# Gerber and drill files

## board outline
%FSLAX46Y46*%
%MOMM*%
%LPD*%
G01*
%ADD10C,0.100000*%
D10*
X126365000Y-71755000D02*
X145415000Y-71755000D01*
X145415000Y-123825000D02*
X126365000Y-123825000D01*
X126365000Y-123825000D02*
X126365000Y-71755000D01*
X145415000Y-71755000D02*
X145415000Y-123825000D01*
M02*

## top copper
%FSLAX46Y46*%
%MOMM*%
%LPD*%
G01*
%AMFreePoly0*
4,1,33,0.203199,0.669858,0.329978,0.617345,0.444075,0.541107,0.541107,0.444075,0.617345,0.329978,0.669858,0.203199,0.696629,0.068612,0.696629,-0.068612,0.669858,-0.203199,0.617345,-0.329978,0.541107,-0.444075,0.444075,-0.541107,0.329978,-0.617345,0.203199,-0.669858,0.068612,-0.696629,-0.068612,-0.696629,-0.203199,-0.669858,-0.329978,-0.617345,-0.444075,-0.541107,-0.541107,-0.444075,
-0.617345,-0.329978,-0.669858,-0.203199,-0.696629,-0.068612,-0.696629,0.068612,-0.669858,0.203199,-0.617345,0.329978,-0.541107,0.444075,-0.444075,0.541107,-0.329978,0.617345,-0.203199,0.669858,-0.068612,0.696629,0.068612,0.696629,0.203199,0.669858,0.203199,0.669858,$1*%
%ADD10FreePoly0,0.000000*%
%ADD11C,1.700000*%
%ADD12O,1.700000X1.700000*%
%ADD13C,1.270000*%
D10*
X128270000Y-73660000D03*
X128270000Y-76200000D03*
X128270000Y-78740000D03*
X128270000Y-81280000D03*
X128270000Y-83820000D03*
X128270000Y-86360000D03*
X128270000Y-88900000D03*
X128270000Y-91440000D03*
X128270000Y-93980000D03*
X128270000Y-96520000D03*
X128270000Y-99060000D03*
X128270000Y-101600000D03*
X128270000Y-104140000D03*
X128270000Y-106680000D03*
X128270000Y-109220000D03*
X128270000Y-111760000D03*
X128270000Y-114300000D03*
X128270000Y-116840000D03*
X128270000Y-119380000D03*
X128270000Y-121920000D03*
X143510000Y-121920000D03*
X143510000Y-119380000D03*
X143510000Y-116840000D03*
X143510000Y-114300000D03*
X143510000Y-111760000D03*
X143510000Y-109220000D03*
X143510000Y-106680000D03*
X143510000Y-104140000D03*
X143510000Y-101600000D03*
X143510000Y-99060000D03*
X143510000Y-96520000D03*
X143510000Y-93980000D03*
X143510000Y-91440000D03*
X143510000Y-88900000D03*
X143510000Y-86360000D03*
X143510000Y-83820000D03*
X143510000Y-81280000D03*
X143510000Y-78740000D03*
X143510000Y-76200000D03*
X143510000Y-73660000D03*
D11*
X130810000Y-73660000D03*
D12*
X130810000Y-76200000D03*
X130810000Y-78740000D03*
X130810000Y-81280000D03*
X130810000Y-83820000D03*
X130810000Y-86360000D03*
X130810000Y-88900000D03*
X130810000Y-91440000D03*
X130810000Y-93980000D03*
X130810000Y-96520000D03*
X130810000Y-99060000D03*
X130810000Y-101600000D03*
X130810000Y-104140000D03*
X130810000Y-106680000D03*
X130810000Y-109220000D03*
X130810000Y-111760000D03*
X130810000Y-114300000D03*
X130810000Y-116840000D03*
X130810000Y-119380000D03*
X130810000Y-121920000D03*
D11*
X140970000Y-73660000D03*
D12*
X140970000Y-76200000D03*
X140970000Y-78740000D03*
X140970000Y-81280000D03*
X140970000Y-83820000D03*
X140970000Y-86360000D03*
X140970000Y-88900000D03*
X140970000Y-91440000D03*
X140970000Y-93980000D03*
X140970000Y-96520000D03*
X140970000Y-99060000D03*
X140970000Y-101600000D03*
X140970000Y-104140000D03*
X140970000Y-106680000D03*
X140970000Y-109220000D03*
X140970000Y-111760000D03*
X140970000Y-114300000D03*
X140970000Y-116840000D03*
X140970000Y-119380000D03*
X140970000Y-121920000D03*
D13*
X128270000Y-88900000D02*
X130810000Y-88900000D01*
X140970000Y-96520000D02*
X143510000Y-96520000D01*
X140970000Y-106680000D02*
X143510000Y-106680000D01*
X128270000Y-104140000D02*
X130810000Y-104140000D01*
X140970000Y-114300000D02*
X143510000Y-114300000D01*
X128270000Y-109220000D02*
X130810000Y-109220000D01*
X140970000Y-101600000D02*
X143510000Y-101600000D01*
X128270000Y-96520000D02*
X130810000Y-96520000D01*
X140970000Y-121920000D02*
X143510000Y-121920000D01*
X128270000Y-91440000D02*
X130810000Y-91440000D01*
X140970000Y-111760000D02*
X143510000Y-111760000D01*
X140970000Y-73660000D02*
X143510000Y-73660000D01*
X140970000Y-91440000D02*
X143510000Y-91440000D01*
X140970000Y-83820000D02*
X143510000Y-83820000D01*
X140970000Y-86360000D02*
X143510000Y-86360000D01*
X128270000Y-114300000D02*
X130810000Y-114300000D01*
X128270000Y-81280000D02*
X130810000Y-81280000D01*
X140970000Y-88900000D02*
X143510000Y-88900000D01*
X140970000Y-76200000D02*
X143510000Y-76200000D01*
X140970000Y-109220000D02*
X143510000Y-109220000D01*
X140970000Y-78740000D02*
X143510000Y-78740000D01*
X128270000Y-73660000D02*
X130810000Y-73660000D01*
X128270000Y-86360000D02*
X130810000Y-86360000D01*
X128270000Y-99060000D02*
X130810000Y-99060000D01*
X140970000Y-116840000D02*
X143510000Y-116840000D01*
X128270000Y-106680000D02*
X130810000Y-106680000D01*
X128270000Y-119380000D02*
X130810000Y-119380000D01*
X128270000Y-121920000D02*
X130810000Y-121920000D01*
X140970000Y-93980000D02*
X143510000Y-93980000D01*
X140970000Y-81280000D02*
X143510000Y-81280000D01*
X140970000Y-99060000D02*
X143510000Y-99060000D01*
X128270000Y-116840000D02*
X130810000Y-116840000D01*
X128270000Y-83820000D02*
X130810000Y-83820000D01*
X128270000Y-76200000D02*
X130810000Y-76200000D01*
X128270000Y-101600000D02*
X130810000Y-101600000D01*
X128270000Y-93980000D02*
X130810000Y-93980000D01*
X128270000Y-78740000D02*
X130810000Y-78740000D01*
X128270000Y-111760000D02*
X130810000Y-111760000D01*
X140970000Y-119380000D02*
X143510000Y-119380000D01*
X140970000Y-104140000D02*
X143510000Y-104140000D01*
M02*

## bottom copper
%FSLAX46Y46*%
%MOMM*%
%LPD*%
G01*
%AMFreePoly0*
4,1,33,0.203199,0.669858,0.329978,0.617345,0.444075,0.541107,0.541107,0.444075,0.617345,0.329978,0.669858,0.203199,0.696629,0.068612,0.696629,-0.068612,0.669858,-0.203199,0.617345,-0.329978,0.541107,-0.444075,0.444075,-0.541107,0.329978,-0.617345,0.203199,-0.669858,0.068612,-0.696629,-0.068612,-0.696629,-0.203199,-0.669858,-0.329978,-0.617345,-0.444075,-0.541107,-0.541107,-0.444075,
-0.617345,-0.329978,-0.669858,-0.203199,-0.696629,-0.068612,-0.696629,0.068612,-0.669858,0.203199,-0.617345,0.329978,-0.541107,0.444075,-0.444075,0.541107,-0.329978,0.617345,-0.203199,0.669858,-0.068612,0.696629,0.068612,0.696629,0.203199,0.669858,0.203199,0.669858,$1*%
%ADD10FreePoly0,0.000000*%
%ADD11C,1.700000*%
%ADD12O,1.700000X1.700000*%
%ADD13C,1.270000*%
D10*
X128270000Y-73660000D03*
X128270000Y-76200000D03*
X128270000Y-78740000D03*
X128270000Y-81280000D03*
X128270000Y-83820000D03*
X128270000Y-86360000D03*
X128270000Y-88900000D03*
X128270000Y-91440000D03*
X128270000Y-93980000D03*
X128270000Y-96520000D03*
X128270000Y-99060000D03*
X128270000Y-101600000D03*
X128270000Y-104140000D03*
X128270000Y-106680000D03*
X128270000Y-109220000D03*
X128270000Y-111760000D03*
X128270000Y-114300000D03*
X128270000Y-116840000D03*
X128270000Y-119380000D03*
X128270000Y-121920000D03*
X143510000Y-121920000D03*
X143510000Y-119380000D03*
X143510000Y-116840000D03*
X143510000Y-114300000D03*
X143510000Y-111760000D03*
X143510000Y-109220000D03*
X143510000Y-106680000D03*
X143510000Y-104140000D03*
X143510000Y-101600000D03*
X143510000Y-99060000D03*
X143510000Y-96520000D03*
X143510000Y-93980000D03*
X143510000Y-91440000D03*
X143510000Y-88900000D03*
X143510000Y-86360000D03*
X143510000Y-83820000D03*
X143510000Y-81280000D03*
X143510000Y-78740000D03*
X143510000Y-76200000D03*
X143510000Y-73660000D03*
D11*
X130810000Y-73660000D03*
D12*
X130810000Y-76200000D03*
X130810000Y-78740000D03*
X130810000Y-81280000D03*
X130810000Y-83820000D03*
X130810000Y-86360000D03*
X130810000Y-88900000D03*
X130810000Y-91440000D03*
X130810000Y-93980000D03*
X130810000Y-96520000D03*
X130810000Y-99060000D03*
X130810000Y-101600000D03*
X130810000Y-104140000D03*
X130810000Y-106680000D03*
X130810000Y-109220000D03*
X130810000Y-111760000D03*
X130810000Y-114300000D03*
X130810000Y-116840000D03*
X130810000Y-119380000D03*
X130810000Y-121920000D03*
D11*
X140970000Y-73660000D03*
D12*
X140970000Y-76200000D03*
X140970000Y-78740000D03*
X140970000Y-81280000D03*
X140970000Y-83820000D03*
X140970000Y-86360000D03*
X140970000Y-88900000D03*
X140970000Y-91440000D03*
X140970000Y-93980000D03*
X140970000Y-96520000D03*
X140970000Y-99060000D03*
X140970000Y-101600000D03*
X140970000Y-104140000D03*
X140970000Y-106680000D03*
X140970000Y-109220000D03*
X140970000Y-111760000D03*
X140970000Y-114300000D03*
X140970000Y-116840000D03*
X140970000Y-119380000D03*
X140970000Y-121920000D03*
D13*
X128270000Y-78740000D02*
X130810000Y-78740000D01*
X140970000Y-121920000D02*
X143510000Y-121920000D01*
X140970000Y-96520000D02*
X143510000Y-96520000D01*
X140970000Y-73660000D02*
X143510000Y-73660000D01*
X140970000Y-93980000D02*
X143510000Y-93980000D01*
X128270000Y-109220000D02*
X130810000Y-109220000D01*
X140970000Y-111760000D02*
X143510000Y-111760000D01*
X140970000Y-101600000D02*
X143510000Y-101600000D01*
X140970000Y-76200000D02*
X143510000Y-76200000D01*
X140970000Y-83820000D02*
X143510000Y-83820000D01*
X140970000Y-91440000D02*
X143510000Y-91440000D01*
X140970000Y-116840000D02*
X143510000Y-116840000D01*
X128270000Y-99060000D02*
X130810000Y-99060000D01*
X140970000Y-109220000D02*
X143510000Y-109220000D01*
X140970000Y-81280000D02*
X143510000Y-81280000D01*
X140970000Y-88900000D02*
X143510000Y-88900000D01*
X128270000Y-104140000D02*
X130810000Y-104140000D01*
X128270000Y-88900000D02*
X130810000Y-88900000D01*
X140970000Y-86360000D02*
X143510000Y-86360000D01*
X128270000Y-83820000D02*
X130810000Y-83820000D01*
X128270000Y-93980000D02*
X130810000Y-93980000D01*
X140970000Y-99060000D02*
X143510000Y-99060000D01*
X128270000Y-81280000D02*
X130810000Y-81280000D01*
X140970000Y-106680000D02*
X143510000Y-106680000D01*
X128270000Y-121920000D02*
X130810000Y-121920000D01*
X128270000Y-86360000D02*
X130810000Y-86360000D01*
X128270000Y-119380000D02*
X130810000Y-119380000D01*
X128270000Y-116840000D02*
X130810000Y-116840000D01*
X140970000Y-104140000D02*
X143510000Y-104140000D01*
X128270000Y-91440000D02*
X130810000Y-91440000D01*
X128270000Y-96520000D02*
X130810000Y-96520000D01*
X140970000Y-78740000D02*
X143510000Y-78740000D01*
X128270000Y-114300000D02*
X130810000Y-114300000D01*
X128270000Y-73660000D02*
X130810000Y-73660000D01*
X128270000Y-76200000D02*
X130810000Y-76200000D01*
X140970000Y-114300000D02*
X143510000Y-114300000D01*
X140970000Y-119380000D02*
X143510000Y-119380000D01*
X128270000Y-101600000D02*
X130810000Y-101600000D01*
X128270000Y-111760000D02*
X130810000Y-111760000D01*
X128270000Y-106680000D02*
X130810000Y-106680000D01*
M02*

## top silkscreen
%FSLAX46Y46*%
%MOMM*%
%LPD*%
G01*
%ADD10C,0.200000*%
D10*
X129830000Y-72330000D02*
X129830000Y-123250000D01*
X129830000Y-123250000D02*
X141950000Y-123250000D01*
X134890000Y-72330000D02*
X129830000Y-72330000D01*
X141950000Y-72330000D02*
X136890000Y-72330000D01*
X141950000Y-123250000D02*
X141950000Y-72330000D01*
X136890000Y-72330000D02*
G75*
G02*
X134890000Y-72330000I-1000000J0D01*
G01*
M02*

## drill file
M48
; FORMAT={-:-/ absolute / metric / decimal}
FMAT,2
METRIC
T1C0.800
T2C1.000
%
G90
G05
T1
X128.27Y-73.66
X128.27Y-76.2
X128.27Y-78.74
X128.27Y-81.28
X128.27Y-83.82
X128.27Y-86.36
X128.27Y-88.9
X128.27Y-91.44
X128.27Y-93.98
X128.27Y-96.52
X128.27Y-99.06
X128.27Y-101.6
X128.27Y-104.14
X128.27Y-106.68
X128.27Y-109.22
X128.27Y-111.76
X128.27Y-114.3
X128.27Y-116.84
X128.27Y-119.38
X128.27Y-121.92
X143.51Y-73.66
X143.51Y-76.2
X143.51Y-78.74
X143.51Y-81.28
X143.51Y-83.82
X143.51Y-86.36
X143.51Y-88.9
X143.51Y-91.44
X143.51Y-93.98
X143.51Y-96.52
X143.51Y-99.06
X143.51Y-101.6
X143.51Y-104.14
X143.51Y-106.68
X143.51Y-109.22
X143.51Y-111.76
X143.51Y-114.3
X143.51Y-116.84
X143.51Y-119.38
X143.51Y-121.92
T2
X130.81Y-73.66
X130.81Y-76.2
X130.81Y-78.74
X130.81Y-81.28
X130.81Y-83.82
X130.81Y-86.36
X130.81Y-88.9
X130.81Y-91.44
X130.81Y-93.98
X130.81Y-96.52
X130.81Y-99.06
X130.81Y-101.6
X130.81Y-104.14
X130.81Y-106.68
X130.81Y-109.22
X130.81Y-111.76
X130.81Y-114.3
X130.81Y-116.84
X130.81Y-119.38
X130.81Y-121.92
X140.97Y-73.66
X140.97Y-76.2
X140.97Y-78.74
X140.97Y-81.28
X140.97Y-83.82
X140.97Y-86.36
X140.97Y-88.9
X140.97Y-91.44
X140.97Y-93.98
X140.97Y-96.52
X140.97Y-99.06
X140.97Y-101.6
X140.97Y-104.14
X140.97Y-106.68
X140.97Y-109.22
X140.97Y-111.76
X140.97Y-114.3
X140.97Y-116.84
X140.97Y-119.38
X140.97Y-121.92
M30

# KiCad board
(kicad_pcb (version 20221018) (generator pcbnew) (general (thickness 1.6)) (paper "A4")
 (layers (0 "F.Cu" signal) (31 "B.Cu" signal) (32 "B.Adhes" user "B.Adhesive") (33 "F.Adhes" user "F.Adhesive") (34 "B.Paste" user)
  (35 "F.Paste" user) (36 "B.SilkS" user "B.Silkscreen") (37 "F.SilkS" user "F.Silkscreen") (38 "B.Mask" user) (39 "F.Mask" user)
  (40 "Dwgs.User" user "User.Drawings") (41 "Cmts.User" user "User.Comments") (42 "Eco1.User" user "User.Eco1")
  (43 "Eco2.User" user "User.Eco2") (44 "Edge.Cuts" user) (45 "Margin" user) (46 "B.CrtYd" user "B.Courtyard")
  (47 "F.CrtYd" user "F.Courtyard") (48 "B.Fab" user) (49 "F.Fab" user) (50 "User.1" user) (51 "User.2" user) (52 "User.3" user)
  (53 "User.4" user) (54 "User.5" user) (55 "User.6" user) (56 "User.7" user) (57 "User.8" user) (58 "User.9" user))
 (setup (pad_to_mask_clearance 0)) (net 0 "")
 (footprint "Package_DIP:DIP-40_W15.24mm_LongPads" (layer "F.Cu") (at 128.27 73.66)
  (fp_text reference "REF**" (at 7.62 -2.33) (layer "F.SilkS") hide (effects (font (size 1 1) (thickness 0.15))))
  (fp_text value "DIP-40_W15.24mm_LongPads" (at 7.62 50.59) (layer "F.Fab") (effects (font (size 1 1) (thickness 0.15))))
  (fp_line (start 1.56 -1.33) (end 1.56 49.59) (stroke (width 0.2) (type solid)) (layer "F.SilkS"))
  (fp_line (start 1.56 49.59) (end 13.68 49.59) (stroke (width 0.2) (type solid)) (layer "F.SilkS"))
  (fp_line (start 6.62 -1.33) (end 1.56 -1.33) (stroke (width 0.2) (type solid)) (layer "F.SilkS"))
  (fp_line (start 13.68 -1.33) (end 8.62 -1.33) (stroke (width 0.2) (type solid)) (layer "F.SilkS"))
  (fp_line (start 13.68 49.59) (end 13.68 -1.33) (stroke (width 0.2) (type solid)) (layer "F.SilkS"))
  (fp_arc (start 8.62 -1.33) (mid 7.62 -0.33) (end 6.62 -1.33) (stroke (width 0.2) (type solid)) (layer "F.SilkS"))
  (pad "1" thru_hole custom (at 0 0) (size 1.4 1.4) (drill 0.8) (layers "*.Cu" "*.Mask") (zone_connect 0) (thermal_bridge_angle 90)
   (options (clearance outline) (anchor circle)) (primitives))
  (pad "2" thru_hole custom (at 0 2.54) (size 1.4 1.4) (drill 0.8) (layers "*.Cu" "*.Mask") (zone_connect 0) (thermal_bridge_angle 90)
   (options (clearance outline) (anchor circle)) (primitives))
  (pad "3" thru_hole custom (at 0 5.08) (size 1.4 1.4) (drill 0.8) (layers "*.Cu" "*.Mask") (zone_connect 0) (thermal_bridge_angle 90)
   (options (clearance outline) (anchor circle)) (primitives))
  (pad "4" thru_hole custom (at 0 7.62) (size 1.4 1.4) (drill 0.8) (layers "*.Cu" "*.Mask") (zone_connect 0) (thermal_bridge_angle 90)
   (options (clearance outline) (anchor circle)) (primitives))
  (pad "5" thru_hole custom (at 0 10.16) (size 1.4 1.4) (drill 0.8) (layers "*.Cu" "*.Mask") (zone_connect 0) (thermal_bridge_angle 90)
   (options (clearance outline) (anchor circle)) (primitives))
  (pad "6" thru_hole custom (at 0 12.7) (size 1.4 1.4) (drill 0.8) (layers "*.Cu" "*.Mask") (zone_connect 0) (thermal_bridge_angle 90)
   (options (clearance outline) (anchor circle)) (primitives))
  (pad "7" thru_hole custom (at 0 15.24) (size 1.4 1.4) (drill 0.8) (layers "*.Cu" "*.Mask") (zone_connect 0) (thermal_bridge_angle 90)
   (options (clearance outline) (anchor circle)) (primitives))
  (pad "8" thru_hole custom (at 0 17.78) (size 1.4 1.4) (drill 0.8) (layers "*.Cu" "*.Mask") (zone_connect 0) (thermal_bridge_angle 90)
   (options (clearance outline) (anchor circle)) (primitives))
  (pad "9" thru_hole custom (at 0 20.32) (size 1.4 1.4) (drill 0.8) (layers "*.Cu" "*.Mask") (zone_connect 0) (thermal_bridge_angle 90)
   (options (clearance outline) (anchor circle)) (primitives))
  (pad "10" thru_hole custom (at 0 22.86) (size 1.4 1.4) (drill 0.8) (layers "*.Cu" "*.Mask") (zone_connect 0) (thermal_bridge_angle 90)
   (options (clearance outline) (anchor circle)) (primitives))
  (pad "11" thru_hole custom (at 0 25.4) (size 1.4 1.4) (drill 0.8) (layers "*.Cu" "*.Mask") (zone_connect 0) (thermal_bridge_angle 90)
   (options (clearance outline) (anchor circle)) (primitives))
  (pad "12" thru_hole custom (at 0 27.94) (size 1.4 1.4) (drill 0.8) (layers "*.Cu" "*.Mask") (zone_connect 0) (thermal_bridge_angle 90)
   (options (clearance outline) (anchor circle)) (primitives))
  (pad "13" thru_hole custom (at 0 30.48) (size 1.4 1.4) (drill 0.8) (layers "*.Cu" "*.Mask") (zone_connect 0) (thermal_bridge_angle 90)
   (options (clearance outline) (anchor circle)) (primitives))
  (pad "14" thru_hole custom (at 0 33.02) (size 1.4 1.4) (drill 0.8) (layers "*.Cu" "*.Mask") (zone_connect 0) (thermal_bridge_angle 90)
   (options (clearance outline) (anchor circle)) (primitives))
  (pad "15" thru_hole custom (at 0 35.56) (size 1.4 1.4) (drill 0.8) (layers "*.Cu" "*.Mask") (zone_connect 0) (thermal_bridge_angle 90)
   (options (clearance outline) (anchor circle)) (primitives))
  (pad "16" thru_hole custom (at 0 38.1) (size 1.4 1.4) (drill 0.8) (layers "*.Cu" "*.Mask") (zone_connect 0) (thermal_bridge_angle 90)
   (options (clearance outline) (anchor circle)) (primitives))
  (pad "17" thru_hole custom (at 0 40.64) (size 1.4 1.4) (drill 0.8) (layers "*.Cu" "*.Mask") (zone_connect 0) (thermal_bridge_angle 90)
   (options (clearance outline) (anchor circle)) (primitives))
  (pad "18" thru_hole custom (at 0 43.18) (size 1.4 1.4) (drill 0.8) (layers "*.Cu" "*.Mask") (zone_connect 0) (thermal_bridge_angle 90)
   (options (clearance outline) (anchor circle)) (primitives))
  (pad "19" thru_hole custom (at 0 45.72) (size 1.4 1.4) (drill 0.8) (layers "*.Cu" "*.Mask") (zone_connect 0) (thermal_bridge_angle 90)
   (options (clearance outline) (anchor circle)) (primitives))
  (pad "20" thru_hole custom (at 0 48.26) (size 1.4 1.4) (drill 0.8) (layers "*.Cu" "*.Mask") (zone_connect 0) (thermal_bridge_angle 90)
   (options (clearance outline) (anchor circle)) (primitives))
  (pad "21" thru_hole custom (at 15.24 48.26) (size 1.4 1.4) (drill 0.8) (layers "*.Cu" "*.Mask") (zone_connect 0) (thermal_bridge_angle 90)
   (options (clearance outline) (anchor circle)) (primitives))
  (pad "22" thru_hole custom (at 15.24 45.72) (size 1.4 1.4) (drill 0.8) (layers "*.Cu" "*.Mask") (zone_connect 0) (thermal_bridge_angle 90)
   (options (clearance outline) (anchor circle)) (primitives))
  (pad "23" thru_hole custom (at 15.24 43.18) (size 1.4 1.4) (drill 0.8) (layers "*.Cu" "*.Mask") (zone_connect 0) (thermal_bridge_angle 90)
   (options (clearance outline) (anchor circle)) (primitives))
  (pad "24" thru_hole custom (at 15.24 40.64) (size 1.4 1.4) (drill 0.8) (layers "*.Cu" "*.Mask") (zone_connect 0) (thermal_bridge_angle 90)
   (options (clearance outline) (anchor circle)) (primitives))
  (pad "25" thru_hole custom (at 15.24 38.1) (size 1.4 1.4) (drill 0.8) (layers "*.Cu" "*.Mask") (zone_connect 0) (thermal_bridge_angle 90)
   (options (clearance outline) (anchor circle)) (primitives))
  (pad "26" thru_hole custom (at 15.24 35.56) (size 1.4 1.4) (drill 0.8) (layers "*.Cu" "*.Mask") (zone_connect 0) (thermal_bridge_angle 90)
   (options (clearance outline) (anchor circle)) (primitives))
  (pad "27" thru_hole custom (at 15.24 33.02) (size 1.4 1.4) (drill 0.8) (layers "*.Cu" "*.Mask") (zone_connect 0) (thermal_bridge_angle 90)
   (options (clearance outline) (anchor circle)) (primitives))
  (pad "28" thru_hole custom (at 15.24 30.48) (size 1.4 1.4) (drill 0.8) (layers "*.Cu" "*.Mask") (zone_connect 0) (thermal_bridge_angle 90)
   (options (clearance outline) (anchor circle)) (primitives))
  (pad "29" thru_hole custom (at 15.24 27.94) (size 1.4 1.4) (drill 0.8) (layers "*.Cu" "*.Mask") (zone_connect 0) (thermal_bridge_angle 90)
   (options (clearance outline) (anchor circle)) (primitives))
  (pad "30" thru_hole custom (at 15.24 25.4) (size 1.4 1.4) (drill 0.8) (layers "*.Cu" "*.Mask") (zone_connect 0) (thermal_bridge_angle 90)
   (options (clearance outline) (anchor circle)) (primitives))
  (pad "31" thru_hole custom (at 15.24 22.86) (size 1.4 1.4) (drill 0.8) (layers "*.Cu" "*.Mask") (zone_connect 0) (thermal_bridge_angle 90)
   (options (clearance outline) (anchor circle)) (primitives))
  (pad "32" thru_hole custom (at 15.24 20.32) (size 1.4 1.4) (drill 0.8) (layers "*.Cu" "*.Mask") (zone_connect 0) (thermal_bridge_angle 90)
   (options (clearance outline) (anchor circle)) (primitives))
  (pad "33" thru_hole custom (at 15.24 17.78) (size 1.4 1.4) (drill 0.8) (layers "*.Cu" "*.Mask") (zone_connect 0) (thermal_bridge_angle 90)
   (options (clearance outline) (anchor circle)) (primitives))
  (pad "34" thru_hole custom (at 15.24 15.24) (size 1.4 1.4) (drill 0.8) (layers "*.Cu" "*.Mask") (zone_connect 0) (thermal_bridge_angle 90)
   (options (clearance outline) (anchor circle)) (primitives))
  (pad "35" thru_hole custom (at 15.24 12.7) (size 1.4 1.4) (drill 0.8) (layers "*.Cu" "*.Mask") (zone_connect 0) (thermal_bridge_angle 90)
   (options (clearance outline) (anchor circle)) (primitives))
  (pad "36" thru_hole custom (at 15.24 10.16) (size 1.4 1.4) (drill 0.8) (layers "*.Cu" "*.Mask") (zone_connect 0) (thermal_bridge_angle 90)
   (options (clearance outline) (anchor circle)) (primitives))
  (pad "37" thru_hole custom (at 15.24 7.62) (size 1.4 1.4) (drill 0.8) (layers "*.Cu" "*.Mask") (zone_connect 0) (thermal_bridge_angle 90)
   (options (clearance outline) (anchor circle)) (primitives))
  (pad "38" thru_hole custom (at 15.24 5.08) (size 1.4 1.4) (drill 0.8) (layers "*.Cu" "*.Mask") (zone_connect 0) (thermal_bridge_angle 90)
   (options (clearance outline) (anchor circle)) (primitives))
  (pad "39" thru_hole custom (at 15.24 2.54) (size 1.4 1.4) (drill 0.8) (layers "*.Cu" "*.Mask") (zone_connect 0) (thermal_bridge_angle 90)
   (options (clearance outline) (anchor circle)) (primitives))
  (pad "40" thru_hole custom (at 15.24 0) (size 1.4 1.4) (drill 0.8) (layers "*.Cu" "*.Mask") (zone_connect 0) (thermal_bridge_angle 90)
   (options (clearance outline) (anchor circle)) (primitives)))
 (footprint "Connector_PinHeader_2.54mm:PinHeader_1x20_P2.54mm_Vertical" (layer "B.Cu") (at 130.81 73.66 180)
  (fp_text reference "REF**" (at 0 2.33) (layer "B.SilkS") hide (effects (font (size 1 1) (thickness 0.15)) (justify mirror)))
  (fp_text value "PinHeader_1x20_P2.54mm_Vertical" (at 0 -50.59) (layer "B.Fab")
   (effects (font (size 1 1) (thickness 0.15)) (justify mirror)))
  (pad "1" thru_hole circle (at 0 0 180) (size 1.7 1.7) (drill 1) (layers "*.Cu" "*.Mask"))
  (pad "2" thru_hole oval (at 0 -2.54 180) (size 1.7 1.7) (drill 1) (layers "*.Cu" "*.Mask"))
  (pad "3" thru_hole oval (at 0 -5.08 180) (size 1.7 1.7) (drill 1) (layers "*.Cu" "*.Mask"))
  (pad "4" thru_hole oval (at 0 -7.62 180) (size 1.7 1.7) (drill 1) (layers "*.Cu" "*.Mask"))
  (pad "5" thru_hole oval (at 0 -10.16 180) (size 1.7 1.7) (drill 1) (layers "*.Cu" "*.Mask"))
  (pad "6" thru_hole oval (at 0 -12.7 180) (size 1.7 1.7) (drill 1) (layers "*.Cu" "*.Mask"))
  (pad "7" thru_hole oval (at 0 -15.24 180) (size 1.7 1.7) (drill 1) (layers "*.Cu" "*.Mask"))
  (pad "8" thru_hole oval (at 0 -17.78 180) (size 1.7 1.7) (drill 1) (layers "*.Cu" "*.Mask"))
  (pad "9" thru_hole oval (at 0 -20.32 180) (size 1.7 1.7) (drill 1) (layers "*.Cu" "*.Mask"))
  (pad "10" thru_hole oval (at 0 -22.86 180) (size 1.7 1.7) (drill 1) (layers "*.Cu" "*.Mask"))
  (pad "11" thru_hole oval (at 0 -25.4 180) (size 1.7 1.7) (drill 1) (layers "*.Cu" "*.Mask"))
  (pad "12" thru_hole oval (at 0 -27.94 180) (size 1.7 1.7) (drill 1) (layers "*.Cu" "*.Mask"))
  (pad "13" thru_hole oval (at 0 -30.48 180) (size 1.7 1.7) (drill 1) (layers "*.Cu" "*.Mask"))
  (pad "14" thru_hole oval (at 0 -33.02 180) (size 1.7 1.7) (drill 1) (layers "*.Cu" "*.Mask"))
  (pad "15" thru_hole oval (at 0 -35.56 180) (size 1.7 1.7) (drill 1) (layers "*.Cu" "*.Mask"))
  (pad "16" thru_hole oval (at 0 -38.1 180) (size 1.7 1.7) (drill 1) (layers "*.Cu" "*.Mask"))
  (pad "17" thru_hole oval (at 0 -40.64 180) (size 1.7 1.7) (drill 1) (layers "*.Cu" "*.Mask"))
  (pad "18" thru_hole oval (at 0 -43.18 180) (size 1.7 1.7) (drill 1) (layers "*.Cu" "*.Mask"))
  (pad "19" thru_hole oval (at 0 -45.72 180) (size 1.7 1.7) (drill 1) (layers "*.Cu" "*.Mask"))
  (pad "20" thru_hole oval (at 0 -48.26 180) (size 1.7 1.7) (drill 1) (layers "*.Cu" "*.Mask")))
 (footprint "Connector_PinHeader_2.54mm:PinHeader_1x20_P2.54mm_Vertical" (layer "B.Cu") (at 140.97 73.66 180)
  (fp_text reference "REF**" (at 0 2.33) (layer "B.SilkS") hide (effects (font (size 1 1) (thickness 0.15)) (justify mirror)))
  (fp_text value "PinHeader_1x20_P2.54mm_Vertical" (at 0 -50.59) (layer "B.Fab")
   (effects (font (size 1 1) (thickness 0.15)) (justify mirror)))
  (pad "1" thru_hole circle (at 0 0 180) (size 1.7 1.7) (drill 1) (layers "*.Cu" "*.Mask"))
  (pad "2" thru_hole oval (at 0 -2.54 180) (size 1.7 1.7) (drill 1) (layers "*.Cu" "*.Mask"))
  (pad "3" thru_hole oval (at 0 -5.08 180) (size 1.7 1.7) (drill 1) (layers "*.Cu" "*.Mask"))
  (pad "4" thru_hole oval (at 0 -7.62 180) (size 1.7 1.7) (drill 1) (layers "*.Cu" "*.Mask"))
  (pad "5" thru_hole oval (at 0 -10.16 180) (size 1.7 1.7) (drill 1) (layers "*.Cu" "*.Mask"))
  (pad "6" thru_hole oval (at 0 -12.7 180) (size 1.7 1.7) (drill 1) (layers "*.Cu" "*.Mask"))
  (pad "7" thru_hole oval (at 0 -15.24 180) (size 1.7 1.7) (drill 1) (layers "*.Cu" "*.Mask"))
  (pad "8" thru_hole oval (at 0 -17.78 180) (size 1.7 1.7) (drill 1) (layers "*.Cu" "*.Mask"))
  (pad "9" thru_hole oval (at 0 -20.32 180) (size 1.7 1.7) (drill 1) (layers "*.Cu" "*.Mask"))
  (pad "10" thru_hole oval (at 0 -22.86 180) (size 1.7 1.7) (drill 1) (layers "*.Cu" "*.Mask"))
  (pad "11" thru_hole oval (at 0 -25.4 180) (size 1.7 1.7) (drill 1) (layers "*.Cu" "*.Mask"))
  (pad "12" thru_hole oval (at 0 -27.94 180) (size 1.7 1.7) (drill 1) (layers "*.Cu" "*.Mask"))
  (pad "13" thru_hole oval (at 0 -30.48 180) (size 1.7 1.7) (drill 1) (layers "*.Cu" "*.Mask"))
  (pad "14" thru_hole oval (at 0 -33.02 180) (size 1.7 1.7) (drill 1) (layers "*.Cu" "*.Mask"))
  (pad "15" thru_hole oval (at 0 -35.56 180) (size 1.7 1.7) (drill 1) (layers "*.Cu" "*.Mask"))
  (pad "16" thru_hole oval (at 0 -38.1 180) (size 1.7 1.7) (drill 1) (layers "*.Cu" "*.Mask"))
  (pad "17" thru_hole oval (at 0 -40.64 180) (size 1.7 1.7) (drill 1) (layers "*.Cu" "*.Mask"))
  (pad "18" thru_hole oval (at 0 -43.18 180) (size 1.7 1.7) (drill 1) (layers "*.Cu" "*.Mask"))
  (pad "19" thru_hole oval (at 0 -45.72 180) (size 1.7 1.7) (drill 1) (layers "*.Cu" "*.Mask"))
  (pad "20" thru_hole oval (at 0 -48.26 180) (size 1.7 1.7) (drill 1) (layers "*.Cu" "*.Mask")))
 (gr_line (start 126.365 71.755) (end 145.415 71.755) (stroke (width 0.1) (type default)) (layer "Edge.Cuts"))
 (gr_line (start 145.415 123.825) (end 126.365 123.825) (stroke (width 0.1) (type default)) (layer "Edge.Cuts"))
 (gr_line (start 126.365 123.825) (end 126.365 71.755) (stroke (width 0.1) (type default)) (layer "Edge.Cuts"))
 (gr_line (start 145.415 71.755) (end 145.415 123.825) (stroke (width 0.1) (type default)) (layer "Edge.Cuts"))
 (segment (start 128.27 88.9) (end 130.81 88.9) (width 1.27) (layer "F.Cu") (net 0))
 (segment (start 140.97 96.52) (end 143.51 96.52) (width 1.27) (layer "F.Cu") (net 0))
 (segment (start 140.97 106.68) (end 143.51 106.68) (width 1.27) (layer "F.Cu") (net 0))
 (segment (start 128.27 104.14) (end 130.81 104.14) (width 1.27) (layer "F.Cu") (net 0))
 (segment (start 140.97 114.3) (end 143.51 114.3) (width 1.27) (layer "F.Cu") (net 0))
 (segment (start 128.27 109.22) (end 130.81 109.22) (width 1.27) (layer "F.Cu") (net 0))
 (segment (start 140.97 101.6) (end 143.51 101.6) (width 1.27) (layer "F.Cu") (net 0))
 (segment (start 128.27 96.52) (end 130.81 96.52) (width 1.27) (layer "F.Cu") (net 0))
 (segment (start 140.97 121.92) (end 143.51 121.92) (width 1.27) (layer "F.Cu") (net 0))
 (segment (start 128.27 91.44) (end 130.81 91.44) (width 1.27) (layer "F.Cu") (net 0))
 (segment (start 140.97 111.76) (end 143.51 111.76) (width 1.27) (layer "F.Cu") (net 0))
 (segment (start 140.97 73.66) (end 143.51 73.66) (width 1.27) (layer "F.Cu") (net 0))
 (segment (start 140.97 91.44) (end 143.51 91.44) (width 1.27) (layer "F.Cu") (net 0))
 (segment (start 140.97 83.82) (end 143.51 83.82) (width 1.27) (layer "F.Cu") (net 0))
 (segment (start 140.97 86.36) (end 143.51 86.36) (width 1.27) (layer "F.Cu") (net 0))
 (segment (start 128.27 114.3) (end 130.81 114.3) (width 1.27) (layer "F.Cu") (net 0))
 (segment (start 128.27 81.28) (end 130.81 81.28) (width 1.27) (layer "F.Cu") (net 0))
 (segment (start 140.97 88.9) (end 143.51 88.9) (width 1.27) (layer "F.Cu") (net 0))
 (segment (start 140.97 76.2) (end 143.51 76.2) (width 1.27) (layer "F.Cu") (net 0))
 (segment (start 140.97 109.22) (end 143.51 109.22) (width 1.27) (layer "F.Cu") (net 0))
 (segment (start 140.97 78.74) (end 143.51 78.74) (width 1.27) (layer "F.Cu") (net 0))
 (segment (start 128.27 73.66) (end 130.81 73.66) (width 1.27) (layer "F.Cu") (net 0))
 (segment (start 128.27 86.36) (end 130.81 86.36) (width 1.27) (layer "F.Cu") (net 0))
 (segment (start 128.27 99.06) (end 130.81 99.06) (width 1.27) (layer "F.Cu") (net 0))
 (segment (start 140.97 116.84) (end 143.51 116.84) (width 1.27) (layer "F.Cu") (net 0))
 (segment (start 128.27 106.68) (end 130.81 106.68) (width 1.27) (layer "F.Cu") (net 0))
 (segment (start 128.27 119.38) (end 130.81 119.38) (width 1.27) (layer "F.Cu") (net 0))
 (segment (start 128.27 121.92) (end 130.81 121.92) (width 1.27) (layer "F.Cu") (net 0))
 (segment (start 140.97 93.98) (end 143.51 93.98) (width 1.27) (layer "F.Cu") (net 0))
 (segment (start 140.97 81.28) (end 143.51 81.28) (width 1.27) (layer "F.Cu") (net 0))
 (segment (start 140.97 99.06) (end 143.51 99.06) (width 1.27) (layer "F.Cu") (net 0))
 (segment (start 128.27 116.84) (end 130.81 116.84) (width 1.27) (layer "F.Cu") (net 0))
 (segment (start 128.27 83.82) (end 130.81 83.82) (width 1.27) (layer "F.Cu") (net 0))
 (segment (start 128.27 76.2) (end 130.81 76.2) (width 1.27) (layer "F.Cu") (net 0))
 (segment (start 128.27 101.6) (end 130.81 101.6) (width 1.27) (layer "F.Cu") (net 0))
 (segment (start 128.27 93.98) (end 130.81 93.98) (width 1.27) (layer "F.Cu") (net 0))
 (segment (start 128.27 78.74) (end 130.81 78.74) (width 1.27) (layer "F.Cu") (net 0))
 (segment (start 128.27 111.76) (end 130.81 111.76) (width 1.27) (layer "F.Cu") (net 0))
 (segment (start 140.97 119.38) (end 143.51 119.38) (width 1.27) (layer "F.Cu") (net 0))
 (segment (start 140.97 104.14) (end 143.51 104.14) (width 1.27) (layer "F.Cu") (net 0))
 (segment (start 128.27 78.74) (end 130.81 78.74) (width 1.27) (layer "B.Cu") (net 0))
 (segment (start 140.97 121.92) (end 143.51 121.92) (width 1.27) (layer "B.Cu") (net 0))
 (segment (start 140.97 96.52) (end 143.51 96.52) (width 1.27) (layer "B.Cu") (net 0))
 (segment (start 140.97 73.66) (end 143.51 73.66) (width 1.27) (layer "B.Cu") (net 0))
 (segment (start 140.97 93.98) (end 143.51 93.98) (width 1.27) (layer "B.Cu") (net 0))
 (segment (start 128.27 109.22) (end 130.81 109.22) (width 1.27) (layer "B.Cu") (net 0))
 (segment (start 140.97 111.76) (end 143.51 111.76) (width 1.27) (layer "B.Cu") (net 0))
 (segment (start 140.97 101.6) (end 143.51 101.6) (width 1.27) (layer "B.Cu") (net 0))
 (segment (start 140.97 76.2) (end 143.51 76.2) (width 1.27) (layer "B.Cu") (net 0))
 (segment (start 140.97 83.82) (end 143.51 83.82) (width 1.27) (layer "B.Cu") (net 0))
 (segment (start 140.97 91.44) (end 143.51 91.44) (width 1.27) (layer "B.Cu") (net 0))
 (segment (start 140.97 116.84) (end 143.51 116.84) (width 1.27) (layer "B.Cu") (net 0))
 (segment (start 128.27 99.06) (end 130.81 99.06) (width 1.27) (layer "B.Cu") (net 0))
 (segment (start 140.97 109.22) (end 143.51 109.22) (width 1.27) (layer "B.Cu") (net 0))
 (segment (start 140.97 81.28) (end 143.51 81.28) (width 1.27) (layer "B.Cu") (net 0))
 (segment (start 140.97 88.9) (end 143.51 88.9) (width 1.27) (layer "B.Cu") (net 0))
 (segment (start 128.27 104.14) (end 130.81 104.14) (width 1.27) (layer "B.Cu") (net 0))
 (segment (start 128.27 88.9) (end 130.81 88.9) (width 1.27) (layer "B.Cu") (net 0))
 (segment (start 140.97 86.36) (end 143.51 86.36) (width 1.27) (layer "B.Cu") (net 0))
 (segment (start 128.27 83.82) (end 130.81 83.82) (width 1.27) (layer "B.Cu") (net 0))
 (segment (start 128.27 93.98) (end 130.81 93.98) (width 1.27) (layer "B.Cu") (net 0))
 (segment (start 140.97 99.06) (end 143.51 99.06) (width 1.27) (layer "B.Cu") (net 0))
 (segment (start 128.27 81.28) (end 130.81 81.28) (width 1.27) (layer "B.Cu") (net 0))
 (segment (start 140.97 106.68) (end 143.51 106.68) (width 1.27) (layer "B.Cu") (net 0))
 (segment (start 128.27 121.92) (end 130.81 121.92) (width 1.27) (layer "B.Cu") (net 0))
 (segment (start 128.27 86.36) (end 130.81 86.36) (width 1.27) (layer "B.Cu") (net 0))
 (segment (start 128.27 119.38) (end 130.81 119.38) (width 1.27) (layer "B.Cu") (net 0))
 (segment (start 128.27 116.84) (end 130.81 116.84) (width 1.27) (layer "B.Cu") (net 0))
 (segment (start 140.97 104.14) (end 143.51 104.14) (width 1.27) (layer "B.Cu") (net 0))
 (segment (start 128.27 91.44) (end 130.81 91.44) (width 1.27) (layer "B.Cu") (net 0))
 (segment (start 128.27 96.52) (end 130.81 96.52) (width 1.27) (layer "B.Cu") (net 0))
 (segment (start 140.97 78.74) (end 143.51 78.74) (width 1.27) (layer "B.Cu") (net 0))
 (segment (start 128.27 114.3) (end 130.81 114.3) (width 1.27) (layer "B.Cu") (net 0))
 (segment (start 128.27 73.66) (end 130.81 73.66) (width 1.27) (layer "B.Cu") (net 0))
 (segment (start 128.27 76.2) (end 130.81 76.2) (width 1.27) (layer "B.Cu") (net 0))
 (segment (start 140.97 114.3) (end 143.51 114.3) (width 1.27) (layer "B.Cu") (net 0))
 (segment (start 140.97 119.38) (end 143.51 119.38) (width 1.27) (layer "B.Cu") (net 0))
 (segment (start 128.27 101.6) (end 130.81 101.6) (width 1.27) (layer "B.Cu") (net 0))
 (segment (start 128.27 111.76) (end 130.81 111.76) (width 1.27) (layer "B.Cu") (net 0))
 (segment (start 128.27 106.68) (end 130.81 106.68) (width 1.27) (layer "B.Cu") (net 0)))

